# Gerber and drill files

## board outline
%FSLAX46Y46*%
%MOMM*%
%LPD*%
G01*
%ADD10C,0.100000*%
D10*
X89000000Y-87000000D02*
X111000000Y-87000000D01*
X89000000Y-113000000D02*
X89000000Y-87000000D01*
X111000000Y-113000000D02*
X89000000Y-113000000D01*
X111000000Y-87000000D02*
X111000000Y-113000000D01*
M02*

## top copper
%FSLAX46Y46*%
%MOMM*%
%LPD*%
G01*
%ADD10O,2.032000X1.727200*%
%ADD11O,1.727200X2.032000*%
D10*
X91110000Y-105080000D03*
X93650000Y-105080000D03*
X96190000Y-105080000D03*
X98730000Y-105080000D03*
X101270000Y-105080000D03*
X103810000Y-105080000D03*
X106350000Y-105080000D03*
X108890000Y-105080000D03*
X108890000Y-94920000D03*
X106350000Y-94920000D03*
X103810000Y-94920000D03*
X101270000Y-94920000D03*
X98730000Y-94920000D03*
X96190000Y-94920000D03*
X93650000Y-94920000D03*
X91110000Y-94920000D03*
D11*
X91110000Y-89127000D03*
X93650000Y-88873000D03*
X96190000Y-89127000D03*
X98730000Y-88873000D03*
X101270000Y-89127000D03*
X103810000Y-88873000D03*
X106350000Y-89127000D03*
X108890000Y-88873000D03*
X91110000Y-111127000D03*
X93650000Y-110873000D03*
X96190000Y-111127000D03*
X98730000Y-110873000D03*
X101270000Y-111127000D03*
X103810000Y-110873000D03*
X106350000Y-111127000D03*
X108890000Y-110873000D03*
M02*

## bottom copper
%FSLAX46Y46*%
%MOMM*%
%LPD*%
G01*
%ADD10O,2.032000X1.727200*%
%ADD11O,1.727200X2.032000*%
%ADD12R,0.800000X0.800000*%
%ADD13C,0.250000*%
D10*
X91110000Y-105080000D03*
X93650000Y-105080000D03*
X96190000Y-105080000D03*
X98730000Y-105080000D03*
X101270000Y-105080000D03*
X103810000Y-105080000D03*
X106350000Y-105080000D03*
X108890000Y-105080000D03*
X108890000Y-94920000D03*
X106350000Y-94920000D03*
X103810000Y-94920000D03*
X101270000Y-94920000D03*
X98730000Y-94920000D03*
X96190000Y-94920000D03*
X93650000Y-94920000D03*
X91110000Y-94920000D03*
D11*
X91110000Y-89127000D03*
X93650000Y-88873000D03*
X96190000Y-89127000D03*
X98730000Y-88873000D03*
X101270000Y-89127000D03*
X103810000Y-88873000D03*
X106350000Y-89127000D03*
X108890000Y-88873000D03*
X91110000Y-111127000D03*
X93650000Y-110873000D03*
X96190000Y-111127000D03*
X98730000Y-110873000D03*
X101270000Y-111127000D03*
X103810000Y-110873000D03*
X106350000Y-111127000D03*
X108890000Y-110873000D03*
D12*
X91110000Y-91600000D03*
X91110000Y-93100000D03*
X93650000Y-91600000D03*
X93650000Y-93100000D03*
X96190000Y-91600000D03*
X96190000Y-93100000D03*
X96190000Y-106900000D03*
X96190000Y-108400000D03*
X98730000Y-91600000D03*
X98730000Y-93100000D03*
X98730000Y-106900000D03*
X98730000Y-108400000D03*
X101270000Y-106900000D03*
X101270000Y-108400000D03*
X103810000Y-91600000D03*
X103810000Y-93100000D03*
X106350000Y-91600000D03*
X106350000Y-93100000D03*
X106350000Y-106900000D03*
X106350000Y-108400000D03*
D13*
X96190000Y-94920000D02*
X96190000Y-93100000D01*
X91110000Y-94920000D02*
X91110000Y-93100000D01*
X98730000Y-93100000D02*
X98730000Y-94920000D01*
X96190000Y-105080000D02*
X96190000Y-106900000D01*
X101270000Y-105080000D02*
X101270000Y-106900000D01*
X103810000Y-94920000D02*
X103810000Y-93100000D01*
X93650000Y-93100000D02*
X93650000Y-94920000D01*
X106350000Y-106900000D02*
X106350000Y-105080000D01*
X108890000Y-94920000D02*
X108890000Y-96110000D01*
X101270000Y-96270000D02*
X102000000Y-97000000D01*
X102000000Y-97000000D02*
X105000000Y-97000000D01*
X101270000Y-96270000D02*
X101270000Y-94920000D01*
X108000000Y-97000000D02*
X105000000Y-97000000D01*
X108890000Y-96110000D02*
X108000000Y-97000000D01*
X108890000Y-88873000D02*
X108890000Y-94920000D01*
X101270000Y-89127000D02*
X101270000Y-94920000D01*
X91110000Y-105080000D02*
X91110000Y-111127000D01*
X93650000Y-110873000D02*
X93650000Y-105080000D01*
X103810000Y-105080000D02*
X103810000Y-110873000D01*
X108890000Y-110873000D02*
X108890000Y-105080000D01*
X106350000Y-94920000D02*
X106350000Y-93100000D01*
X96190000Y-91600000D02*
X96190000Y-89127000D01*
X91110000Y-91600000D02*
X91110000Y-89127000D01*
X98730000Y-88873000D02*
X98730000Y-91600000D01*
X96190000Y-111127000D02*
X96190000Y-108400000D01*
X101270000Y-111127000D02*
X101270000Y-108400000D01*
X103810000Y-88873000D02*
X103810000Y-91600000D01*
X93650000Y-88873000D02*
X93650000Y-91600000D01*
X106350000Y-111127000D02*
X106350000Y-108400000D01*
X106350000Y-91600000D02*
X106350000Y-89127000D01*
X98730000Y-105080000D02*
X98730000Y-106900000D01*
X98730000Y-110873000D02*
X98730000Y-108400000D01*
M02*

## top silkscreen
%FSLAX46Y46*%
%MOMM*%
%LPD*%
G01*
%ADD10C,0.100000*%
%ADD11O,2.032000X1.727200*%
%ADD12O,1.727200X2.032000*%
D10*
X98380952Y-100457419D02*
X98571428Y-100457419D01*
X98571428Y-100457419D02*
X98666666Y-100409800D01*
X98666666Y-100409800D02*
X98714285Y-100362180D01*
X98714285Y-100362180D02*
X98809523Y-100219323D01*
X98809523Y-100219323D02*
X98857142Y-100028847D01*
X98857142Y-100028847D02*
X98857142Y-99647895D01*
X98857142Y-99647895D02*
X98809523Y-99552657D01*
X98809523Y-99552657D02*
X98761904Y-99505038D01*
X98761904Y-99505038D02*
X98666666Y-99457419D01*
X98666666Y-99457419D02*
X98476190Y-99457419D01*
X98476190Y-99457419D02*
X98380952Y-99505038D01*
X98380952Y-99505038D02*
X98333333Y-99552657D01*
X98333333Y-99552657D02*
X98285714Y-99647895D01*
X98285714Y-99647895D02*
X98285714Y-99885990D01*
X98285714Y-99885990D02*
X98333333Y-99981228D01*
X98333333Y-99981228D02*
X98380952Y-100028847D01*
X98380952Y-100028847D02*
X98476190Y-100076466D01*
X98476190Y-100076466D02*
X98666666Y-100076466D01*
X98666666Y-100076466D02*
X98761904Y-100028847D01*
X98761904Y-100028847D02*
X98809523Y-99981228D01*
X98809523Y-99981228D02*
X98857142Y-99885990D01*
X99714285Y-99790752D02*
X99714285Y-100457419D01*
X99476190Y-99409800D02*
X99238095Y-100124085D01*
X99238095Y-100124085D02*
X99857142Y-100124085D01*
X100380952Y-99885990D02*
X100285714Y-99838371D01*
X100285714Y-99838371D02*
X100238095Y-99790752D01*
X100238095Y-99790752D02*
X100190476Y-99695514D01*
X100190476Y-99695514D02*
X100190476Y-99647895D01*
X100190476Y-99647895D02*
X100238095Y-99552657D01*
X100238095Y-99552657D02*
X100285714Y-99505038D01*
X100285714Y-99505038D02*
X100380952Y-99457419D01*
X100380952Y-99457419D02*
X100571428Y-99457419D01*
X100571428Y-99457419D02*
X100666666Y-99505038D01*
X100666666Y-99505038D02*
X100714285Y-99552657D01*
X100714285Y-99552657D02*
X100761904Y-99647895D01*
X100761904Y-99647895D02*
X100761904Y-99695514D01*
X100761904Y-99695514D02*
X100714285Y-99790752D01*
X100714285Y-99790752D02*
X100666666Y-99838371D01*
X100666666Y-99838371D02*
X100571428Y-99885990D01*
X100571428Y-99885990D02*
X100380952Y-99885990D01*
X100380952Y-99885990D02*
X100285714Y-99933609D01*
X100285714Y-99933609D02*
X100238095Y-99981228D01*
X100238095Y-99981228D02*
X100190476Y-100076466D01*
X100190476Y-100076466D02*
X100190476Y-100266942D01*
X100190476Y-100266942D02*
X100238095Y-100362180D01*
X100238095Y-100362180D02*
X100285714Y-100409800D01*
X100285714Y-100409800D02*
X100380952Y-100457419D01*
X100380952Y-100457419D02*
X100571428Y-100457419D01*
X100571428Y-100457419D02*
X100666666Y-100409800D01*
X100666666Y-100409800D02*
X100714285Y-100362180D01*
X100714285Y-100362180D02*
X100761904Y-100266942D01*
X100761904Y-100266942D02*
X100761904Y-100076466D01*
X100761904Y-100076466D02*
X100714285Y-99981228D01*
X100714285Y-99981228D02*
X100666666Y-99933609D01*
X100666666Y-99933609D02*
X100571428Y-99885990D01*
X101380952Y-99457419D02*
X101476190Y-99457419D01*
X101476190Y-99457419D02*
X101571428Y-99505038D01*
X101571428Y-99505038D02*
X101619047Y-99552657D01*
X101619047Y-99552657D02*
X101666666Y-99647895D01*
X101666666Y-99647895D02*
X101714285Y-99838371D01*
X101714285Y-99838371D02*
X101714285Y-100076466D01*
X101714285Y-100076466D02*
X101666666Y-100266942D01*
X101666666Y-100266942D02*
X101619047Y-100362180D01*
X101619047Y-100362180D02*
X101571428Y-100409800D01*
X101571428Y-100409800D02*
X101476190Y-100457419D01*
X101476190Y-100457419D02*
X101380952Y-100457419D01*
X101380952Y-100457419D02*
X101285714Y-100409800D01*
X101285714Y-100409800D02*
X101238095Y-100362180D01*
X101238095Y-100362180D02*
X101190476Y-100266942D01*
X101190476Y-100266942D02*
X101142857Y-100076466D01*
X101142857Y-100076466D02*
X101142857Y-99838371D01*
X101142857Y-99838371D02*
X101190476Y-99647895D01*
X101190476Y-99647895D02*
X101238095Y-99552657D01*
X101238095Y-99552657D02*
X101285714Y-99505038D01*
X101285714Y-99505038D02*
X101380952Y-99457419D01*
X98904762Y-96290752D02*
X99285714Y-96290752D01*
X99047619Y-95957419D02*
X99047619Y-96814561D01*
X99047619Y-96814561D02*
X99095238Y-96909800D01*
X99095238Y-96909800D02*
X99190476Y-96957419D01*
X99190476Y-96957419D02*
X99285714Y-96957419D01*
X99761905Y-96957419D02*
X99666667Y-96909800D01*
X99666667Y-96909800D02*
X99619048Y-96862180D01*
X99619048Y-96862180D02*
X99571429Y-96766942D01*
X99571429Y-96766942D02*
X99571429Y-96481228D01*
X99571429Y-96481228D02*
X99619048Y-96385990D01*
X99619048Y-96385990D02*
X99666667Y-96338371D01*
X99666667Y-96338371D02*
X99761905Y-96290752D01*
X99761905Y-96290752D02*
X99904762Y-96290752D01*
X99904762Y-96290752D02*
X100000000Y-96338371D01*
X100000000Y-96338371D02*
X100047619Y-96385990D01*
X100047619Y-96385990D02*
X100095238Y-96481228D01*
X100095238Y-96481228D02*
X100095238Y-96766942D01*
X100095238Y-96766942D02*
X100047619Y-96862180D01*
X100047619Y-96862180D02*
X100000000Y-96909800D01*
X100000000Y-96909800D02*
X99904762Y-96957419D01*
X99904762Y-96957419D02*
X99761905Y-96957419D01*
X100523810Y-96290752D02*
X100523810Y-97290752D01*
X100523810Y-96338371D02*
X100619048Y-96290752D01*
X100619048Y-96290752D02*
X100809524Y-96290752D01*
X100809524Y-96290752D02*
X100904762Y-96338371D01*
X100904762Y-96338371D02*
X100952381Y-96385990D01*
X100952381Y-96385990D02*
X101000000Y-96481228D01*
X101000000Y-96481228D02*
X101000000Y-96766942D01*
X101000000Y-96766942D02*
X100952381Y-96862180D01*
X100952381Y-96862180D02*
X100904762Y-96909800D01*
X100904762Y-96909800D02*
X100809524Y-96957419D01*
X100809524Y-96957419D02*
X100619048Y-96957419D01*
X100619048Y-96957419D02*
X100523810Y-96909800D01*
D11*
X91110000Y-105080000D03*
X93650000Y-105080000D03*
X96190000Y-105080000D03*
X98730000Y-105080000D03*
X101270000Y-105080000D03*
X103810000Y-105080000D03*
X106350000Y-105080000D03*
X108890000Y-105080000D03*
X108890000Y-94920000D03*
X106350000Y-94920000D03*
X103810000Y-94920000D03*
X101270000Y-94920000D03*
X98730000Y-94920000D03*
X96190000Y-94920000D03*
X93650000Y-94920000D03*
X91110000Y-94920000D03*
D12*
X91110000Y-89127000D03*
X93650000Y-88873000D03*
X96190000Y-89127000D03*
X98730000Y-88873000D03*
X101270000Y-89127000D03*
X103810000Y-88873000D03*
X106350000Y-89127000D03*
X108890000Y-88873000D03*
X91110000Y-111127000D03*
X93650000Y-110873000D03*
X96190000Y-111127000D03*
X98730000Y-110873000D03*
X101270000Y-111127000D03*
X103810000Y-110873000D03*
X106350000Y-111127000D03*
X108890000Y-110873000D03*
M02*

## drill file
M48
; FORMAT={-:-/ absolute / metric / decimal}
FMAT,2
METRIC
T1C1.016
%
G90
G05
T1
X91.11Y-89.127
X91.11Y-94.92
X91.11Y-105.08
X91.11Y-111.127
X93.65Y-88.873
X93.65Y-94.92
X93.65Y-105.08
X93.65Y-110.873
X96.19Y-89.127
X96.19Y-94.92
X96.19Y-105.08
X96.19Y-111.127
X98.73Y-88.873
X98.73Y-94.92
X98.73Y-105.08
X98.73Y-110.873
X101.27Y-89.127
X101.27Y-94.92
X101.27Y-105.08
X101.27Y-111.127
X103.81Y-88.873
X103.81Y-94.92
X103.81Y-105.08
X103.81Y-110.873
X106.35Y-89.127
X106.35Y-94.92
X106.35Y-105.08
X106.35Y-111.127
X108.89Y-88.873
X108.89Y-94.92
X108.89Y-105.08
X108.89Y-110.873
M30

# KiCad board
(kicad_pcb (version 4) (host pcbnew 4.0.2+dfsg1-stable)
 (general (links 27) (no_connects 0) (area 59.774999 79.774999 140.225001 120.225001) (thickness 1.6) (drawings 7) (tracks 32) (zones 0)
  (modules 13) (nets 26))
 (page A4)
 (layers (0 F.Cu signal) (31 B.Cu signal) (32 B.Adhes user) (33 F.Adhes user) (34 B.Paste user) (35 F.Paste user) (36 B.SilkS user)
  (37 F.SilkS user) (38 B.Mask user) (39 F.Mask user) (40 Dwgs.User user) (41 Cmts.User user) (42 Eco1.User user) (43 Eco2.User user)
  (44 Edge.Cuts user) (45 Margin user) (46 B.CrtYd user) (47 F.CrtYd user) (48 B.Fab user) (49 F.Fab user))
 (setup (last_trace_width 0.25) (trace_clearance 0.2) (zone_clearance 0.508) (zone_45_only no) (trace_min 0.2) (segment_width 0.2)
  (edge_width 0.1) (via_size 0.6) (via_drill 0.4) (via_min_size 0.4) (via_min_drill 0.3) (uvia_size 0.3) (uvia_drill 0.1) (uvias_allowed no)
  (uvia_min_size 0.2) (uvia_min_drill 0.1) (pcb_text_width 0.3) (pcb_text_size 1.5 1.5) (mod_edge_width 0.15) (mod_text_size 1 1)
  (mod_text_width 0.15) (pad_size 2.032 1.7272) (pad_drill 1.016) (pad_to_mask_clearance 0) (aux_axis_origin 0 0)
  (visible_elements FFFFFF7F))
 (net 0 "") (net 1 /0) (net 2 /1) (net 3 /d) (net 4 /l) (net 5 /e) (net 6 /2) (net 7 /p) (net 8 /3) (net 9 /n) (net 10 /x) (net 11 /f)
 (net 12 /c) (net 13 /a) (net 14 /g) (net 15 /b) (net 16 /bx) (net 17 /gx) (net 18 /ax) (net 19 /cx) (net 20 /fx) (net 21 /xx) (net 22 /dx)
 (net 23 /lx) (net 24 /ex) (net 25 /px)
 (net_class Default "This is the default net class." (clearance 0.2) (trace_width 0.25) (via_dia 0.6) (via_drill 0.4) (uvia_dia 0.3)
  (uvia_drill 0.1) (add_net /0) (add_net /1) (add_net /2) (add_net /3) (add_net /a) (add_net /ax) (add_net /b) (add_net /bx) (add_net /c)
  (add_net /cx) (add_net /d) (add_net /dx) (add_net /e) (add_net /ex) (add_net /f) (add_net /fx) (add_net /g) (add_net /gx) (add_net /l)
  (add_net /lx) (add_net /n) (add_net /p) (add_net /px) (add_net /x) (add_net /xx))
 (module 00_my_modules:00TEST (layer F.Cu) (at 100 100)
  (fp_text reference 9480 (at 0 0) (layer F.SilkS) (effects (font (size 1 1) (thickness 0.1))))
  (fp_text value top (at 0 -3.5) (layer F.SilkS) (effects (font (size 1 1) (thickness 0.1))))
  (pad 0 thru_hole oval (at -8.89 5.08) (size 2.032 1.7272) (drill 1.016) (layers *.Cu *.Mask F.SilkS) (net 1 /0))
  (pad 1 thru_hole oval (at -6.35 5.08) (size 2.032 1.7272) (drill 1.016) (layers *.Cu *.Mask F.SilkS) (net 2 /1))
  (pad D thru_hole oval (at -3.81 5.08) (size 2.032 1.7272) (drill 1.016) (layers *.Cu *.Mask F.SilkS) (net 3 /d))
  (pad L thru_hole oval (at -1.27 5.08) (size 2.032 1.7272) (drill 1.016) (layers *.Cu *.Mask F.SilkS) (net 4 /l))
  (pad E thru_hole oval (at 1.27 5.08) (size 2.032 1.7272) (drill 1.016) (layers *.Cu *.Mask F.SilkS) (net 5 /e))
  (pad 2 thru_hole oval (at 3.81 5.08) (size 2.032 1.7272) (drill 1.016) (layers *.Cu *.Mask F.SilkS) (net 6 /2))
  (pad P thru_hole oval (at 6.35 5.08) (size 2.032 1.7272) (drill 1.016) (layers *.Cu *.Mask F.SilkS) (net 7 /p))
  (pad 3 thru_hole oval (at 8.89 5.08) (size 2.032 1.7272) (drill 1.016) (layers *.Cu *.Mask F.SilkS) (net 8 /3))
  (pad N thru_hole oval (at 8.89 -5.08) (size 2.032 1.7272) (drill 1.016) (layers *.Cu *.Mask F.SilkS) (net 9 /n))
  (pad X thru_hole oval (at 6.35 -5.08) (size 2.032 1.7272) (drill 1.016) (layers *.Cu *.Mask F.SilkS) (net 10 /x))
  (pad F thru_hole oval (at 3.81 -5.08) (size 2.032 1.7272) (drill 1.016) (layers *.Cu *.Mask F.SilkS) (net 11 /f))
  (pad N thru_hole oval (at 1.27 -5.08) (size 2.032 1.7272) (drill 1.016) (layers *.Cu *.Mask F.SilkS) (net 9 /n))
  (pad C thru_hole oval (at -1.27 -5.08) (size 2.032 1.7272) (drill 1.016) (layers *.Cu *.Mask F.SilkS) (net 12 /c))
  (pad A thru_hole oval (at -3.81 -5.08) (size 2.032 1.7272) (drill 1.016) (layers *.Cu *.Mask F.SilkS) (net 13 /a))
  (pad G thru_hole oval (at -6.35 -5.08) (size 2.032 1.7272) (drill 1.016) (layers *.Cu *.Mask F.SilkS) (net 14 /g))
  (pad B thru_hole oval (at -8.89 -5.08) (size 2.032 1.7272) (drill 1.016) (layers *.Cu *.Mask F.SilkS) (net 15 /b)))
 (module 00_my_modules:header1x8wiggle (layer F.Cu) (at 100 89 90)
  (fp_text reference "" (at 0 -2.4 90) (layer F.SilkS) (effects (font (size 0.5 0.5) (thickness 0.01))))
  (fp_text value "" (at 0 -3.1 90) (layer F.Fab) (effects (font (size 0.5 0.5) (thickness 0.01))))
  (pad BX thru_hole oval (at -0.127 -8.89 90) (size 2.032 1.7272) (drill 1.016) (layers *.Cu *.Mask F.SilkS) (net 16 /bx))
  (pad GX thru_hole oval (at 0.127 -6.35 90) (size 2.032 1.7272) (drill 1.016) (layers *.Cu *.Mask F.SilkS) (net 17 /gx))
  (pad AX thru_hole oval (at -0.127 -3.81 90) (size 2.032 1.7272) (drill 1.016) (layers *.Cu *.Mask F.SilkS) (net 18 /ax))
  (pad CX thru_hole oval (at 0.127 -1.27 90) (size 2.032 1.7272) (drill 1.016) (layers *.Cu *.Mask F.SilkS) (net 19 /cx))
  (pad N thru_hole oval (at -0.127 1.27 90) (size 2.032 1.7272) (drill 1.016) (layers *.Cu *.Mask F.SilkS) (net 9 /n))
  (pad FX thru_hole oval (at 0.127 3.81 90) (size 2.032 1.7272) (drill 1.016) (layers *.Cu *.Mask F.SilkS) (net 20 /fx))
  (pad XX thru_hole oval (at -0.127 6.35 90) (size 2.032 1.7272) (drill 1.016) (layers *.Cu *.Mask F.SilkS) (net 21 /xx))
  (pad N thru_hole oval (at 0.127 8.89 90) (size 2.032 1.7272) (drill 1.016) (layers *.Cu *.Mask F.SilkS) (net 9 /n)))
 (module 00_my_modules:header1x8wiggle (layer F.Cu) (at 100 111 90)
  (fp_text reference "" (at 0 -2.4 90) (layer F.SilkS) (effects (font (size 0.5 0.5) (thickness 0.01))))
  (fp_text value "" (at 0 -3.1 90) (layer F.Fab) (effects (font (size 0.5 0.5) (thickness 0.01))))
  (pad 0 thru_hole oval (at -0.127 -8.89 90) (size 2.032 1.7272) (drill 1.016) (layers *.Cu *.Mask F.SilkS) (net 1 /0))
  (pad 1 thru_hole oval (at 0.127 -6.35 90) (size 2.032 1.7272) (drill 1.016) (layers *.Cu *.Mask F.SilkS) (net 2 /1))
  (pad DX thru_hole oval (at -0.127 -3.81 90) (size 2.032 1.7272) (drill 1.016) (layers *.Cu *.Mask F.SilkS) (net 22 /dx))
  (pad LX thru_hole oval (at 0.127 -1.27 90) (size 2.032 1.7272) (drill 1.016) (layers *.Cu *.Mask F.SilkS) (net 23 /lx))
  (pad EX thru_hole oval (at -0.127 1.27 90) (size 2.032 1.7272) (drill 1.016) (layers *.Cu *.Mask F.SilkS) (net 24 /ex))
  (pad 2 thru_hole oval (at 0.127 3.81 90) (size 2.032 1.7272) (drill 1.016) (layers *.Cu *.Mask F.SilkS) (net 6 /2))
  (pad PX thru_hole oval (at -0.127 6.35 90) (size 2.032 1.7272) (drill 1.016) (layers *.Cu *.Mask F.SilkS) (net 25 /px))
  (pad 3 thru_hole oval (at 0.127 8.89 90) (size 2.032 1.7272) (drill 1.016) (layers *.Cu *.Mask F.SilkS) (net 8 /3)))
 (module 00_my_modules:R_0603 (layer B.Cu) (at 91.11 92.35 270)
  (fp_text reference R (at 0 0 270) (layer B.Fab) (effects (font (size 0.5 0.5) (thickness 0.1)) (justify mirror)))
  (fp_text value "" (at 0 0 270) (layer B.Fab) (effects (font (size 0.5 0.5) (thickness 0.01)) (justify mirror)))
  (pad BX smd rect (at -0.75 0 270) (size 0.8 0.8) (layers B.Cu B.Paste B.Mask) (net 16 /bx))
  (pad B smd rect (at 0.75 0 270) (size 0.8 0.8) (layers B.Cu B.Paste B.Mask) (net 15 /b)))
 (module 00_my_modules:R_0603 (layer B.Cu) (at 93.65 92.35 270)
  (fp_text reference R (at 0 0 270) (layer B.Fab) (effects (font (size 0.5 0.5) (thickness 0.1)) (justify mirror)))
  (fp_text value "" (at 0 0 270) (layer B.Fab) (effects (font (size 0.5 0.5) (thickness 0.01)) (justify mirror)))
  (pad GX smd rect (at -0.75 0 270) (size 0.8 0.8) (layers B.Cu B.Paste B.Mask) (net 17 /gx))
  (pad G smd rect (at 0.75 0 270) (size 0.8 0.8) (layers B.Cu B.Paste B.Mask) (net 14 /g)))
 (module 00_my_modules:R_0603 (layer B.Cu) (at 96.19 92.35 270)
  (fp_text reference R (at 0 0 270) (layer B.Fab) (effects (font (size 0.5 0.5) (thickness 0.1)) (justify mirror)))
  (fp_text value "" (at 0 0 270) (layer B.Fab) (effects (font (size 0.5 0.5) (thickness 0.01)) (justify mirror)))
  (pad AX smd rect (at -0.75 0 270) (size 0.8 0.8) (layers B.Cu B.Paste B.Mask) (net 18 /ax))
  (pad A smd rect (at 0.75 0 270) (size 0.8 0.8) (layers B.Cu B.Paste B.Mask) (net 13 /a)))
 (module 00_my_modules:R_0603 (layer B.Cu) (at 96.19 107.65 270)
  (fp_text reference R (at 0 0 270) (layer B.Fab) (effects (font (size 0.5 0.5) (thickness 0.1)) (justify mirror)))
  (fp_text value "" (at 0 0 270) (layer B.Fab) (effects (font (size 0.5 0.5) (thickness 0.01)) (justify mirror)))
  (pad D smd rect (at -0.75 0 270) (size 0.8 0.8) (layers B.Cu B.Paste B.Mask) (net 3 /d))
  (pad DX smd rect (at 0.75 0 270) (size 0.8 0.8) (layers B.Cu B.Paste B.Mask) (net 22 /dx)))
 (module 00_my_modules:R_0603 (layer B.Cu) (at 98.73 92.35 270)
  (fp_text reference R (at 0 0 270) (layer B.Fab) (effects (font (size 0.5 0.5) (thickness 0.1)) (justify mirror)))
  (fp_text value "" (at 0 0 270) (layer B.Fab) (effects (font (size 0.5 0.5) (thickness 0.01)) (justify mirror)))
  (pad CX smd rect (at -0.75 0 270) (size 0.8 0.8) (layers B.Cu B.Paste B.Mask) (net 19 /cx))
  (pad C smd rect (at 0.75 0 270) (size 0.8 0.8) (layers B.Cu B.Paste B.Mask) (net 12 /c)))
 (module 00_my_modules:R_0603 (layer B.Cu) (at 98.73 107.65 270)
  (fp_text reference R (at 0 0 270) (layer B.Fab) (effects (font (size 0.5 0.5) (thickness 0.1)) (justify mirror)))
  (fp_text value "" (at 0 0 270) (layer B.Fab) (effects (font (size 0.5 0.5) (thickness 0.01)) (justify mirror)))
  (pad L smd rect (at -0.75 0 270) (size 0.8 0.8) (layers B.Cu B.Paste B.Mask) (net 4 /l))
  (pad LX smd rect (at 0.75 0 270) (size 0.8 0.8) (layers B.Cu B.Paste B.Mask) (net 23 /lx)))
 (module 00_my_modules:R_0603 (layer B.Cu) (at 101.27 107.65 270)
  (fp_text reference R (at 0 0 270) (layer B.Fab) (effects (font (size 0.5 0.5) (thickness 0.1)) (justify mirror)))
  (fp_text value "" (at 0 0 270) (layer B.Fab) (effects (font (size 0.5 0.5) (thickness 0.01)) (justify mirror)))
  (pad E smd rect (at -0.75 0 270) (size 0.8 0.8) (layers B.Cu B.Paste B.Mask) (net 5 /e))
  (pad EX smd rect (at 0.75 0 270) (size 0.8 0.8) (layers B.Cu B.Paste B.Mask) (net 24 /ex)))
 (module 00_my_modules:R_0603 (layer B.Cu) (at 103.81 92.35 270)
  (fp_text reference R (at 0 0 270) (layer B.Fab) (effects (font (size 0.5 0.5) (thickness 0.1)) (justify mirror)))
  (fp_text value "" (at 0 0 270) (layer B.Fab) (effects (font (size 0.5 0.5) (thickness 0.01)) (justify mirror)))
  (pad FX smd rect (at -0.75 0 270) (size 0.8 0.8) (layers B.Cu B.Paste B.Mask) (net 20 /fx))
  (pad F smd rect (at 0.75 0 270) (size 0.8 0.8) (layers B.Cu B.Paste B.Mask) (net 11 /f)))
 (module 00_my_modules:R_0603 (layer B.Cu) (at 106.35 92.35 270)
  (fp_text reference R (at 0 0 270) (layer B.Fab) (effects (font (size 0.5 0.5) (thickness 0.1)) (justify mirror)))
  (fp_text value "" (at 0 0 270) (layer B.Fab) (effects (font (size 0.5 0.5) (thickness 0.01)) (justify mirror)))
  (pad XX smd rect (at -0.75 0 270) (size 0.8 0.8) (layers B.Cu B.Paste B.Mask) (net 21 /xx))
  (pad X smd rect (at 0.75 0 270) (size 0.8 0.8) (layers B.Cu B.Paste B.Mask) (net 10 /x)))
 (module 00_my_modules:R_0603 (layer B.Cu) (at 106.35 107.65 270)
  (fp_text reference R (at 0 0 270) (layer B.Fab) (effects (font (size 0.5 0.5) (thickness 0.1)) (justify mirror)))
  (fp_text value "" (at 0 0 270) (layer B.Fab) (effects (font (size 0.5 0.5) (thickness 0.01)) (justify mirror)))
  (pad P smd rect (at -0.75 0 270) (size 0.8 0.8) (layers B.Cu B.Paste B.Mask) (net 7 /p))
  (pad PX smd rect (at 0.75 0 270) (size 0.8 0.8) (layers B.Cu B.Paste B.Mask) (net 25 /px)))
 (gr_line (start 89 87) (end 111 87) (angle 90) (layer Edge.Cuts) (width 0.1))
 (gr_line (start 89 113) (end 89 87) (angle 90) (layer Edge.Cuts) (width 0.1))
 (gr_line (start 111 113) (end 89 113) (angle 90) (layer Edge.Cuts) (width 0.1))
 (gr_line (start 111 87) (end 111 113) (angle 90) (layer Edge.Cuts) (width 0.1))
 (segment (start 96.19 94.92) (end 96.19 93.1) (width 0.25) (layer B.Cu) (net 13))
 (segment (start 91.11 94.92) (end 91.11 93.1) (width 0.25) (layer B.Cu) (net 15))
 (segment (start 98.73 93.1) (end 98.73 94.92) (width 0.25) (layer B.Cu) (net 12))
 (segment (start 96.19 105.08) (end 96.19 106.9) (width 0.25) (layer B.Cu) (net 3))
 (segment (start 101.27 105.08) (end 101.27 106.9) (width 0.25) (layer B.Cu) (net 5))
 (segment (start 103.81 94.92) (end 103.81 93.1) (width 0.25) (layer B.Cu) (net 11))
 (segment (start 93.65 93.1) (end 93.65 94.92) (width 0.25) (layer B.Cu) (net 14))
 (segment (start 106.35 106.9) (end 106.35 105.08) (width 0.25) (layer B.Cu) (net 7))
 (segment (start 108.89 94.92) (end 108.89 96.11) (width 0.25) (layer B.Cu) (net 9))
 (segment (start 101.27 96.27) (end 102 97) (width 0.25) (layer B.Cu) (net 9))
 (segment (start 102 97) (end 105 97) (width 0.25) (layer B.Cu) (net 9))
 (segment (start 101.27 96.27) (end 101.27 94.92) (width 0.25) (layer B.Cu) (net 9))
 (segment (start 108 97) (end 105 97) (width 0.25) (layer B.Cu) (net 9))
 (segment (start 108.89 96.11) (end 108 97) (width 0.25) (layer B.Cu) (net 9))
 (segment (start 108.89 88.873) (end 108.89 94.92) (width 0.25) (layer B.Cu) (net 9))
 (segment (start 101.27 89.127) (end 101.27 94.92) (width 0.25) (layer B.Cu) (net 9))
 (segment (start 91.11 105.08) (end 91.11 111.127) (width 0.25) (layer B.Cu) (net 1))
 (segment (start 93.65 110.873) (end 93.65 105.08) (width 0.25) (layer B.Cu) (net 2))
 (segment (start 103.81 105.08) (end 103.81 110.873) (width 0.25) (layer B.Cu) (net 6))
 (segment (start 108.89 110.873) (end 108.89 105.08) (width 0.25) (layer B.Cu) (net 8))
 (segment (start 106.35 94.92) (end 106.35 93.1) (width 0.25) (layer B.Cu) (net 10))
 (segment (start 96.19 91.6) (end 96.19 89.127) (width 0.25) (layer B.Cu) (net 18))
 (segment (start 91.11 91.6) (end 91.11 89.127) (width 0.25) (layer B.Cu) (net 16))
 (segment (start 98.73 88.873) (end 98.73 91.6) (width 0.25) (layer B.Cu) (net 19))
 (segment (start 96.19 111.127) (end 96.19 108.4) (width 0.25) (layer B.Cu) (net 22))
 (segment (start 101.27 111.127) (end 101.27 108.4) (width 0.25) (layer B.Cu) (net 24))
 (segment (start 103.81 88.873) (end 103.81 91.6) (width 0.25) (layer B.Cu) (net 20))
 (segment (start 93.65 88.873) (end 93.65 91.6) (width 0.25) (layer B.Cu) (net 17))
 (segment (start 106.35 111.127) (end 106.35 108.4) (width 0.25) (layer B.Cu) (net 25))
 (segment (start 106.35 91.6) (end 106.35 89.127) (width 0.25) (layer B.Cu) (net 21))
 (segment (start 98.73 105.08) (end 98.73 106.9) (width 0.25) (layer B.Cu) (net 4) (status C00000))
 (segment (start 98.73 110.873) (end 98.73 108.4) (width 0.25) (layer B.Cu) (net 23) (status C00000)))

